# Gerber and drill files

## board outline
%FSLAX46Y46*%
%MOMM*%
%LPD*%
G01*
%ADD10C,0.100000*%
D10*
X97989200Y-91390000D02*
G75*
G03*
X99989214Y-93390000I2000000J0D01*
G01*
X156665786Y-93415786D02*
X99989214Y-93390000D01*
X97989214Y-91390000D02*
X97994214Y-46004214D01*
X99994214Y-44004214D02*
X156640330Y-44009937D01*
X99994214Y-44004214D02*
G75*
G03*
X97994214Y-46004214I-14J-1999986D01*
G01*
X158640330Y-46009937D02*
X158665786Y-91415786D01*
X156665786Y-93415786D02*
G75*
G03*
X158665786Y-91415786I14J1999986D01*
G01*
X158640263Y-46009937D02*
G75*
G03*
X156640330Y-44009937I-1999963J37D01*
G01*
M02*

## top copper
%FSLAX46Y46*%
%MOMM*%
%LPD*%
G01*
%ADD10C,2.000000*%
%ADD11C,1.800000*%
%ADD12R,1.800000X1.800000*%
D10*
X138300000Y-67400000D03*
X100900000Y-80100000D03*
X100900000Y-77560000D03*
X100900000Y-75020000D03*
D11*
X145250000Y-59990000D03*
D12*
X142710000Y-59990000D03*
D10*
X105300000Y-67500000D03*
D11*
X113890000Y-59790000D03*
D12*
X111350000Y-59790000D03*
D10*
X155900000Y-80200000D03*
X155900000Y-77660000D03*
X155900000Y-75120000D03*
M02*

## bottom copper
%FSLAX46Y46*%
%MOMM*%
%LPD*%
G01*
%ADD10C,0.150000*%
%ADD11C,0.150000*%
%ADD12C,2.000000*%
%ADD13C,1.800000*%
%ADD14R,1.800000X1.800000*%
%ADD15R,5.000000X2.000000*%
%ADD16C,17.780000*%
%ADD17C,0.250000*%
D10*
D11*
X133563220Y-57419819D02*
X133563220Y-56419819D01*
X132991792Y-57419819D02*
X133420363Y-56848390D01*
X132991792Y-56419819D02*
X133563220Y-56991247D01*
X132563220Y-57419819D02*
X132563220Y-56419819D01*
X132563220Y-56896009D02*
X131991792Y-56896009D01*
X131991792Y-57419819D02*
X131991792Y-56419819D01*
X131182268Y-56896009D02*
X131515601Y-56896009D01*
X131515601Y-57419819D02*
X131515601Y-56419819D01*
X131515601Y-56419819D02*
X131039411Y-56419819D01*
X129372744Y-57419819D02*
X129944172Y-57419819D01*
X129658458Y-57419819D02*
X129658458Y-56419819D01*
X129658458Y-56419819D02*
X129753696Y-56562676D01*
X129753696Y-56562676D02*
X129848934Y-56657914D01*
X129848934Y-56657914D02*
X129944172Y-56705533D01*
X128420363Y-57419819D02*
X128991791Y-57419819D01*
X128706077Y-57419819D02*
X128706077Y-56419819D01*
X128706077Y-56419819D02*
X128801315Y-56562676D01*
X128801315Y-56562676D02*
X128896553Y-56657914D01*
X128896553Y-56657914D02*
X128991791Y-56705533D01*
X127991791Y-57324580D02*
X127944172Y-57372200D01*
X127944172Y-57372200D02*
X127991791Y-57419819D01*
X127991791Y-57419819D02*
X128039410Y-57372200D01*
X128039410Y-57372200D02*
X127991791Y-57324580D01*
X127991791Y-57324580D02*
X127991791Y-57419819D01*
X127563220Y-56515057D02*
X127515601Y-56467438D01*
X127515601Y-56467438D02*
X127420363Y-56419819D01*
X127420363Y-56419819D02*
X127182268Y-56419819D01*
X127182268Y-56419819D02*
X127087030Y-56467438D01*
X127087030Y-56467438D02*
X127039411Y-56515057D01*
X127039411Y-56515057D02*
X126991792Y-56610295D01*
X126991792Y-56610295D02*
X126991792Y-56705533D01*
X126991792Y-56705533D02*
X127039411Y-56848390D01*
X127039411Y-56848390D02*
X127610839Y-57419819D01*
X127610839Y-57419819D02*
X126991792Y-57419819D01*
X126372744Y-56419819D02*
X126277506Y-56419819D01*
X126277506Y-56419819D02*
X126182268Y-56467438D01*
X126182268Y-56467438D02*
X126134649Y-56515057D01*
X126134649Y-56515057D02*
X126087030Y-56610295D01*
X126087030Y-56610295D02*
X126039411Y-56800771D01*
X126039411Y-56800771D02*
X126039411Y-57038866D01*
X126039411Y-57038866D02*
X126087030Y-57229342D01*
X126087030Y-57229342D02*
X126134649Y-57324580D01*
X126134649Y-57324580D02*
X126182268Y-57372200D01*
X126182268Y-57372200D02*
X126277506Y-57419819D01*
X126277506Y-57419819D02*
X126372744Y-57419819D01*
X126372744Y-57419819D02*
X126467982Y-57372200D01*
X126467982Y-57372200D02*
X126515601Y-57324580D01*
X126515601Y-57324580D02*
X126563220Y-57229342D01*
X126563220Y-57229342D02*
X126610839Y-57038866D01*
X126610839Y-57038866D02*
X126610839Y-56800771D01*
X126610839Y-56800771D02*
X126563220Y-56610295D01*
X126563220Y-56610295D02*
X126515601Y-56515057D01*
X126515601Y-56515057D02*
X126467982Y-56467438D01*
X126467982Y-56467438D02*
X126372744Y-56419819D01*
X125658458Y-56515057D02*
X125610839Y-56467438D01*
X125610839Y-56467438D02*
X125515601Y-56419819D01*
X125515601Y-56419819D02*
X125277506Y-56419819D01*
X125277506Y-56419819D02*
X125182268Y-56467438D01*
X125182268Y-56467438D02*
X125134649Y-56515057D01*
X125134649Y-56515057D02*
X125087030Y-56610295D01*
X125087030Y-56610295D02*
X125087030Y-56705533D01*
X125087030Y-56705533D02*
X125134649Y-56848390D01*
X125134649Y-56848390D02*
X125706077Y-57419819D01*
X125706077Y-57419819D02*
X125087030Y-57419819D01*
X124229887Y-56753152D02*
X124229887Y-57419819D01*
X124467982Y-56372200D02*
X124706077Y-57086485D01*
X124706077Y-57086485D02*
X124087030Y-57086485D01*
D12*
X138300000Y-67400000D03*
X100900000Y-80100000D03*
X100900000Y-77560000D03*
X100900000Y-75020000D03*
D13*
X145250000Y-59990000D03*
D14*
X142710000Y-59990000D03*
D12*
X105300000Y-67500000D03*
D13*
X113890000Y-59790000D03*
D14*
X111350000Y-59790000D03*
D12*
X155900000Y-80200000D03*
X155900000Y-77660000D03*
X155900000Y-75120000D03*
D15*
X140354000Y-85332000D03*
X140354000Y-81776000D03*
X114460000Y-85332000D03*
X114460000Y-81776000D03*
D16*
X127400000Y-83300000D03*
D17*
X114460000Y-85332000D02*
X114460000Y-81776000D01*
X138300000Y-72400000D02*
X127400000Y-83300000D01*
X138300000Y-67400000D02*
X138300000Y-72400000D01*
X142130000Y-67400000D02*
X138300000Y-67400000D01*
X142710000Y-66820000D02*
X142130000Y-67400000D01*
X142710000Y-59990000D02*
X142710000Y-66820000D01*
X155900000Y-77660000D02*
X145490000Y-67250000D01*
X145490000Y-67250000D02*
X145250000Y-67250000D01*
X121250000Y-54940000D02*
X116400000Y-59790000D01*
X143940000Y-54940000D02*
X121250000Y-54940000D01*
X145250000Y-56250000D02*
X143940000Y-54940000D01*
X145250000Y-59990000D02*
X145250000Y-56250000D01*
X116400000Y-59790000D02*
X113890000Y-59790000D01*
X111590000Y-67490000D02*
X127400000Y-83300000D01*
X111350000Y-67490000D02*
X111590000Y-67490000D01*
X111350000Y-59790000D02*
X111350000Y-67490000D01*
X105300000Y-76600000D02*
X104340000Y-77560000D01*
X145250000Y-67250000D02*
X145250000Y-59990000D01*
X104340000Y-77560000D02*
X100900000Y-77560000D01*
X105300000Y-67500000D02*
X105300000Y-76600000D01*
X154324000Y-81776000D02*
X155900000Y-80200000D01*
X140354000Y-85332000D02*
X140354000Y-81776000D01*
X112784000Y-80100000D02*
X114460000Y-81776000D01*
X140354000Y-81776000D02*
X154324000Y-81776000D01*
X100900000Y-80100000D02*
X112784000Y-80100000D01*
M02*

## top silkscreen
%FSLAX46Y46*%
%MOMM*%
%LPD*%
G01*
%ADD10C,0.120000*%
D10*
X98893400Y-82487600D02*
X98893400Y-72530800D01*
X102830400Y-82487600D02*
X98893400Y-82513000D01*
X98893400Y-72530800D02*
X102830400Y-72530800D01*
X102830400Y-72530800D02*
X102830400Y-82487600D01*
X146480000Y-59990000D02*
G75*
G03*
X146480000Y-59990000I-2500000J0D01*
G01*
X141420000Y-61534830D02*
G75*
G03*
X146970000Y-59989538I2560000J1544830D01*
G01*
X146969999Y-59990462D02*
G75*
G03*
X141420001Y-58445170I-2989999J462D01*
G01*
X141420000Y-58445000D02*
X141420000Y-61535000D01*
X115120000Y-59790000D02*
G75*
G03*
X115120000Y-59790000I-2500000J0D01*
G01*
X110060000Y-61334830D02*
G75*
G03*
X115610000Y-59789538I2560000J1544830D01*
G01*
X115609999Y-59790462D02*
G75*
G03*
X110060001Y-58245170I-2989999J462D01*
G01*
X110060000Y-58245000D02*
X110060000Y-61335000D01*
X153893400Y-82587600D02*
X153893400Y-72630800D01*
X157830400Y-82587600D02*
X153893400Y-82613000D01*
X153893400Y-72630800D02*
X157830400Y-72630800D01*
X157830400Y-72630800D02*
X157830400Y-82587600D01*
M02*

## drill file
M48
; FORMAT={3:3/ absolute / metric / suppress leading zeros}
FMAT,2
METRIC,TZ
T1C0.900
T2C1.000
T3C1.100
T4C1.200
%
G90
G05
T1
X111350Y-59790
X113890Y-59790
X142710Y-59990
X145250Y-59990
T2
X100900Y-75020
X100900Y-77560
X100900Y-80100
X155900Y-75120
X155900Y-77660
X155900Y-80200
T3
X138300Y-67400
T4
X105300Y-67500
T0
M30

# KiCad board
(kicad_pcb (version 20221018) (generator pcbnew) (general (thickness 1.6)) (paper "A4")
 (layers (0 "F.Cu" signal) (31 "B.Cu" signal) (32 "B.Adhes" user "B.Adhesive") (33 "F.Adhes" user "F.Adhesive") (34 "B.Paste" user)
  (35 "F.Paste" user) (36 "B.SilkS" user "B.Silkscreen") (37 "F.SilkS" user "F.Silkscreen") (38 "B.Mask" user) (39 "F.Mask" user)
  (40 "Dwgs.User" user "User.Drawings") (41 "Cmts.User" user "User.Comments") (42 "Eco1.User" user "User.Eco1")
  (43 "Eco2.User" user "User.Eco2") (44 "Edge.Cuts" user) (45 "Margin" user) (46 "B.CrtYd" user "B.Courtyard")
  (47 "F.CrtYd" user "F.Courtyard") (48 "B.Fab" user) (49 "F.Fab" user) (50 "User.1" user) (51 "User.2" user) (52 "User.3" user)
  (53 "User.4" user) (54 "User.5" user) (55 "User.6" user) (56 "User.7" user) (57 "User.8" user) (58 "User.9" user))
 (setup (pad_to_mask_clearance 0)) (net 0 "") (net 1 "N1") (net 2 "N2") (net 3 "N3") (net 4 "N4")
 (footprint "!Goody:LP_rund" (layer "F.Cu") (at 138.3 67.4)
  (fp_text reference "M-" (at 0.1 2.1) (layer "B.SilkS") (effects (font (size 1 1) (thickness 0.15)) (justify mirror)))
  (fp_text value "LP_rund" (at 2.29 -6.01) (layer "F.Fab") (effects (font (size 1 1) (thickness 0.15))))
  (pad "1" thru_hole circle (at 0 0) (size 2 2) (drill 1.1) (layers "*.Cu" "*.Mask") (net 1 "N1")))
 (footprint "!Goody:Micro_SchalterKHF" (layer "F.Cu") (at 100.9 80.1 90)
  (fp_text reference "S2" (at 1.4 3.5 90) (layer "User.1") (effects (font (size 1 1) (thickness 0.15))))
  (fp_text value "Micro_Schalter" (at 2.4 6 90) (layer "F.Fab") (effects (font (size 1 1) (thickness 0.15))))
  (fp_line (start -2.3876 -2.0066) (end 7.5692 -2.0066) (stroke (width 0.12) (type solid)) (layer "F.SilkS"))
  (fp_line (start -2.3876 1.9304) (end -2.413 -2.0066) (stroke (width 0.12) (type solid)) (layer "F.SilkS"))
  (fp_line (start 7.5692 -2.0066) (end 7.5692 1.9304) (stroke (width 0.12) (type solid)) (layer "F.SilkS"))
  (fp_line (start 7.5692 1.9304) (end -2.3876 1.9304) (stroke (width 0.12) (type solid)) (layer "F.SilkS"))
  (pad "1" thru_hole circle (at 0 0 90) (size 2 2) (drill 1) (layers "*.Cu" "*.Mask") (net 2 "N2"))
  (pad "2" thru_hole circle (at 2.54 0 90) (size 2 2) (drill 1) (layers "*.Cu" "*.Mask") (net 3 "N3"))
  (pad "3" thru_hole circle (at 5.08 0 90) (size 2 2) (drill 1) (layers "*.Cu" "*.Mask")))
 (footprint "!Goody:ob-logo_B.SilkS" (layer "F.Cu") (at 134.7 66.7)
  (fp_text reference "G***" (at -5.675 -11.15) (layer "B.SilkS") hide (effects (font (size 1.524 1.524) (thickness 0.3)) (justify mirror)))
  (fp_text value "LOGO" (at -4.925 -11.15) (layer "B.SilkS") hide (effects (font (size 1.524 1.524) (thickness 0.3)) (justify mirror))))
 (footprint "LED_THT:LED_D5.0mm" (layer "F.Cu") (at 142.71 59.99)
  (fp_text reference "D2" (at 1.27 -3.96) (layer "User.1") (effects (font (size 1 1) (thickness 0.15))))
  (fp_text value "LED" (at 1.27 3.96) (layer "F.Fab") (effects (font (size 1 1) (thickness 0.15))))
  (fp_line (start -1.29 -1.545) (end -1.29 1.545) (stroke (width 0.12) (type solid)) (layer "F.SilkS"))
  (fp_arc (start -1.29 -1.54483) (mid 2.072002 -2.880433) (end 4.26 0.000462) (stroke (width 0.12) (type solid)) (layer "F.SilkS"))
  (fp_arc (start 4.26 -0.000462) (mid 2.072002 2.880433) (end -1.29 1.54483) (stroke (width 0.12) (type solid)) (layer "F.SilkS"))
  (fp_circle (center 1.27 0) (end 3.77 0) (stroke (width 0.12) (type solid)) (fill none) (layer "F.SilkS"))
  (pad "1" thru_hole rect (at 0 0) (size 1.8 1.8) (drill 0.9) (layers "*.Cu" "*.Mask") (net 1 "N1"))
  (pad "2" thru_hole circle (at 2.54 0) (size 1.8 1.8) (drill 0.9) (layers "*.Cu" "*.Mask") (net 3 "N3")))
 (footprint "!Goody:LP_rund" (layer "F.Cu") (at 105.3 67.5)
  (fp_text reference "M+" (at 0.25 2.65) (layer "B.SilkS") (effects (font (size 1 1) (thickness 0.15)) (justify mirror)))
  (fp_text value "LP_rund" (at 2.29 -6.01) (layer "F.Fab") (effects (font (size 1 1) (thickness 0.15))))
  (pad "1" thru_hole circle (at 0 0) (size 2 2) (drill 1.2) (layers "*.Cu" "*.Mask") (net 3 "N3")))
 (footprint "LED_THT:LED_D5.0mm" (layer "F.Cu") (at 111.35 59.79)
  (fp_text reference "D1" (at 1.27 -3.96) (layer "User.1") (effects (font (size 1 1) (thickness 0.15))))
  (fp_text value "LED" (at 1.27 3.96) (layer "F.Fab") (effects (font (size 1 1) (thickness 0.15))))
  (fp_line (start -1.29 -1.545) (end -1.29 1.545) (stroke (width 0.12) (type solid)) (layer "F.SilkS"))
  (fp_arc (start -1.29 -1.54483) (mid 2.072002 -2.880433) (end 4.26 0.000462) (stroke (width 0.12) (type solid)) (layer "F.SilkS"))
  (fp_arc (start 4.26 -0.000462) (mid 2.072002 2.880433) (end -1.29 1.54483) (stroke (width 0.12) (type solid)) (layer "F.SilkS"))
  (fp_circle (center 1.27 0) (end 3.77 0) (stroke (width 0.12) (type solid)) (fill none) (layer "F.SilkS"))
  (pad "1" thru_hole rect (at 0 0) (size 1.8 1.8) (drill 0.9) (layers "*.Cu" "*.Mask") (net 1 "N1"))
  (pad "2" thru_hole circle (at 2.54 0) (size 1.8 1.8) (drill 0.9) (layers "*.Cu" "*.Mask") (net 3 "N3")))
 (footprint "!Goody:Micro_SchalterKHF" (layer "F.Cu") (at 155.9 80.2 90)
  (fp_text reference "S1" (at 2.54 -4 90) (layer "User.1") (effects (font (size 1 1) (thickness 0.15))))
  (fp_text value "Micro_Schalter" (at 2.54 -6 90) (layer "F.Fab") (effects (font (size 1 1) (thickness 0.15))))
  (fp_line (start -2.3876 -2.0066) (end 7.5692 -2.0066) (stroke (width 0.12) (type solid)) (layer "F.SilkS"))
  (fp_line (start -2.3876 1.9304) (end -2.413 -2.0066) (stroke (width 0.12) (type solid)) (layer "F.SilkS"))
  (fp_line (start 7.5692 -2.0066) (end 7.5692 1.9304) (stroke (width 0.12) (type solid)) (layer "F.SilkS"))
  (fp_line (start 7.5692 1.9304) (end -2.3876 1.9304) (stroke (width 0.12) (type solid)) (layer "F.SilkS"))
  (pad "1" thru_hole circle (at 0 0 90) (size 2 2) (drill 1) (layers "*.Cu" "*.Mask") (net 2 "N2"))
  (pad "2" thru_hole circle (at 2.54 0 90) (size 2 2) (drill 1) (layers "*.Cu" "*.Mask") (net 3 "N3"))
  (pad "3" thru_hole circle (at 5.08 0 90) (size 2 2) (drill 1) (layers "*.Cu" "*.Mask") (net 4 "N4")))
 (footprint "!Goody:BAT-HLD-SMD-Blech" (layer "B.Cu") (at 127.4 83.3 180)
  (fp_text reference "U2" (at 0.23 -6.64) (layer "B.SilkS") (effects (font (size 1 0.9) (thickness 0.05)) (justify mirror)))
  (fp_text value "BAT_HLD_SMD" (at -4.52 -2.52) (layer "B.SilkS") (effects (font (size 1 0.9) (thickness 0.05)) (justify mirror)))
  (pad "" smd rect (at -12.954 -2.032 180) (size 5 2) (layers "B.Cu" "B.Paste" "B.Mask") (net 2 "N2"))
  (pad "" smd rect (at -12.954 1.524 180) (size 5 2) (layers "B.Cu" "B.Paste" "B.Mask") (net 2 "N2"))
  (pad "1" smd rect (at 12.94 -2.032 180) (size 5 2) (layers "B.Cu" "B.Paste" "B.Mask") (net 2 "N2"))
  (pad "1" smd rect (at 12.94 1.524 180) (size 5 2) (layers "B.Cu" "B.Paste" "B.Mask") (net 2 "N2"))
  (pad "2" smd circle (at 0 0 180) (size 17.78 17.78) (layers "B.Cu" "B.Paste" "B.Mask") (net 1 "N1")))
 (gr_arc (start 99.989214 93.39) (mid 98.575 92.804214) (end 97.989214 91.39) (stroke (width 0.1) (type default)) (layer "Edge.Cuts"))
 (gr_line (start 156.665786 93.415786) (end 99.989214 93.39) (stroke (width 0.1) (type default)) (layer "Edge.Cuts"))
 (gr_line (start 97.989214 91.39) (end 97.994214 46.004214) (stroke (width 0.1) (type default)) (layer "Edge.Cuts"))
 (gr_line (start 99.994214 44.004214) (end 156.64033 44.009937) (stroke (width 0.1) (type default)) (layer "Edge.Cuts"))
 (gr_arc (start 97.994214 46.004214) (mid 98.58 44.59) (end 99.994214 44.004214) (stroke (width 0.1) (type default)) (layer "Edge.Cuts"))
 (gr_line (start 158.64033 46.009937) (end 158.665786 91.415786) (stroke (width 0.1) (type default)) (layer "Edge.Cuts"))
 (gr_arc (start 158.665786 91.415786) (mid 158.08 92.83) (end 156.665786 93.415786) (stroke (width 0.1) (type default)) (layer "Edge.Cuts"))
 (gr_arc (start 156.64033 44.009937) (mid 158.054544 44.595723) (end 158.64033 46.009937) (stroke (width 0.1) (type default))
  (layer "Edge.Cuts"))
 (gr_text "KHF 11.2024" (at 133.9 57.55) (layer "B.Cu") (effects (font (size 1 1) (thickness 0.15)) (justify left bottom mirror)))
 (segment (start 142.71 66.82) (end 142.13 67.4) (width 0.25) (layer "B.Cu") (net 1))
 (segment (start 111.35 67.49) (end 111.59 67.49) (width 0.25) (layer "B.Cu") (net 1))
 (segment (start 138.3 72.4) (end 127.4 83.3) (width 0.25) (layer "B.Cu") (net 1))
 (segment (start 138.3 67.4) (end 138.3 72.4) (width 0.25) (layer "B.Cu") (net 1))
 (segment (start 142.71 59.99) (end 142.71 66.82) (width 0.25) (layer "B.Cu") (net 1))
 (segment (start 111.59 67.49) (end 127.4 83.3) (width 0.25) (layer "B.Cu") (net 1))
 (segment (start 142.13 67.4) (end 138.3 67.4) (width 0.25) (layer "B.Cu") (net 1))
 (segment (start 111.35 59.79) (end 111.35 67.49) (width 0.25) (layer "B.Cu") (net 1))
 (segment (start 145.49 67.25) (end 145.25 67.25) (width 0.25) (layer "B.Cu") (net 3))
 (segment (start 105.3 76.6) (end 104.34 77.56) (width 0.25) (layer "B.Cu") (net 3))
 (segment (start 116.4 59.79) (end 113.89 59.79) (width 0.25) (layer "B.Cu") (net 3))
 (segment (start 121.25 54.94) (end 116.4 59.79) (width 0.25) (layer "B.Cu") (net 3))
 (segment (start 145.25 67.25) (end 145.25 59.99) (width 0.25) (layer "B.Cu") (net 3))
 (segment (start 145.25 56.25) (end 143.94 54.94) (width 0.25) (layer "B.Cu") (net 3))
 (segment (start 145.25 59.99) (end 145.25 56.25) (width 0.25) (layer "B.Cu") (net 3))
 (segment (start 104.34 77.56) (end 100.9 77.56) (width 0.25) (layer "B.Cu") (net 3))
 (segment (start 105.3 67.5) (end 105.3 76.6) (width 0.25) (layer "B.Cu") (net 3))
 (segment (start 155.9 77.66) (end 145.49 67.25) (width 0.25) (layer "B.Cu") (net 3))
 (segment (start 143.94 54.94) (end 121.25 54.94) (width 0.25) (layer "B.Cu") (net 3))
 (segment (start 114.46 85.332) (end 114.46 81.776) (width 0.25) (layer "B.Cu") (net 2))
 (segment (start 154.324 81.776) (end 155.9 80.2) (width 0.25) (layer "B.Cu") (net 2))
 (segment (start 140.354 85.332) (end 140.354 81.776) (width 0.25) (layer "B.Cu") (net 2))
 (segment (start 112.784 80.1) (end 114.46 81.776) (width 0.25) (layer "B.Cu") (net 2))
 (segment (start 140.354 81.776) (end 154.324 81.776) (width 0.25) (layer "B.Cu") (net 2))
 (segment (start 100.9 80.1) (end 112.784 80.1) (width 0.25) (layer "B.Cu") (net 2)))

